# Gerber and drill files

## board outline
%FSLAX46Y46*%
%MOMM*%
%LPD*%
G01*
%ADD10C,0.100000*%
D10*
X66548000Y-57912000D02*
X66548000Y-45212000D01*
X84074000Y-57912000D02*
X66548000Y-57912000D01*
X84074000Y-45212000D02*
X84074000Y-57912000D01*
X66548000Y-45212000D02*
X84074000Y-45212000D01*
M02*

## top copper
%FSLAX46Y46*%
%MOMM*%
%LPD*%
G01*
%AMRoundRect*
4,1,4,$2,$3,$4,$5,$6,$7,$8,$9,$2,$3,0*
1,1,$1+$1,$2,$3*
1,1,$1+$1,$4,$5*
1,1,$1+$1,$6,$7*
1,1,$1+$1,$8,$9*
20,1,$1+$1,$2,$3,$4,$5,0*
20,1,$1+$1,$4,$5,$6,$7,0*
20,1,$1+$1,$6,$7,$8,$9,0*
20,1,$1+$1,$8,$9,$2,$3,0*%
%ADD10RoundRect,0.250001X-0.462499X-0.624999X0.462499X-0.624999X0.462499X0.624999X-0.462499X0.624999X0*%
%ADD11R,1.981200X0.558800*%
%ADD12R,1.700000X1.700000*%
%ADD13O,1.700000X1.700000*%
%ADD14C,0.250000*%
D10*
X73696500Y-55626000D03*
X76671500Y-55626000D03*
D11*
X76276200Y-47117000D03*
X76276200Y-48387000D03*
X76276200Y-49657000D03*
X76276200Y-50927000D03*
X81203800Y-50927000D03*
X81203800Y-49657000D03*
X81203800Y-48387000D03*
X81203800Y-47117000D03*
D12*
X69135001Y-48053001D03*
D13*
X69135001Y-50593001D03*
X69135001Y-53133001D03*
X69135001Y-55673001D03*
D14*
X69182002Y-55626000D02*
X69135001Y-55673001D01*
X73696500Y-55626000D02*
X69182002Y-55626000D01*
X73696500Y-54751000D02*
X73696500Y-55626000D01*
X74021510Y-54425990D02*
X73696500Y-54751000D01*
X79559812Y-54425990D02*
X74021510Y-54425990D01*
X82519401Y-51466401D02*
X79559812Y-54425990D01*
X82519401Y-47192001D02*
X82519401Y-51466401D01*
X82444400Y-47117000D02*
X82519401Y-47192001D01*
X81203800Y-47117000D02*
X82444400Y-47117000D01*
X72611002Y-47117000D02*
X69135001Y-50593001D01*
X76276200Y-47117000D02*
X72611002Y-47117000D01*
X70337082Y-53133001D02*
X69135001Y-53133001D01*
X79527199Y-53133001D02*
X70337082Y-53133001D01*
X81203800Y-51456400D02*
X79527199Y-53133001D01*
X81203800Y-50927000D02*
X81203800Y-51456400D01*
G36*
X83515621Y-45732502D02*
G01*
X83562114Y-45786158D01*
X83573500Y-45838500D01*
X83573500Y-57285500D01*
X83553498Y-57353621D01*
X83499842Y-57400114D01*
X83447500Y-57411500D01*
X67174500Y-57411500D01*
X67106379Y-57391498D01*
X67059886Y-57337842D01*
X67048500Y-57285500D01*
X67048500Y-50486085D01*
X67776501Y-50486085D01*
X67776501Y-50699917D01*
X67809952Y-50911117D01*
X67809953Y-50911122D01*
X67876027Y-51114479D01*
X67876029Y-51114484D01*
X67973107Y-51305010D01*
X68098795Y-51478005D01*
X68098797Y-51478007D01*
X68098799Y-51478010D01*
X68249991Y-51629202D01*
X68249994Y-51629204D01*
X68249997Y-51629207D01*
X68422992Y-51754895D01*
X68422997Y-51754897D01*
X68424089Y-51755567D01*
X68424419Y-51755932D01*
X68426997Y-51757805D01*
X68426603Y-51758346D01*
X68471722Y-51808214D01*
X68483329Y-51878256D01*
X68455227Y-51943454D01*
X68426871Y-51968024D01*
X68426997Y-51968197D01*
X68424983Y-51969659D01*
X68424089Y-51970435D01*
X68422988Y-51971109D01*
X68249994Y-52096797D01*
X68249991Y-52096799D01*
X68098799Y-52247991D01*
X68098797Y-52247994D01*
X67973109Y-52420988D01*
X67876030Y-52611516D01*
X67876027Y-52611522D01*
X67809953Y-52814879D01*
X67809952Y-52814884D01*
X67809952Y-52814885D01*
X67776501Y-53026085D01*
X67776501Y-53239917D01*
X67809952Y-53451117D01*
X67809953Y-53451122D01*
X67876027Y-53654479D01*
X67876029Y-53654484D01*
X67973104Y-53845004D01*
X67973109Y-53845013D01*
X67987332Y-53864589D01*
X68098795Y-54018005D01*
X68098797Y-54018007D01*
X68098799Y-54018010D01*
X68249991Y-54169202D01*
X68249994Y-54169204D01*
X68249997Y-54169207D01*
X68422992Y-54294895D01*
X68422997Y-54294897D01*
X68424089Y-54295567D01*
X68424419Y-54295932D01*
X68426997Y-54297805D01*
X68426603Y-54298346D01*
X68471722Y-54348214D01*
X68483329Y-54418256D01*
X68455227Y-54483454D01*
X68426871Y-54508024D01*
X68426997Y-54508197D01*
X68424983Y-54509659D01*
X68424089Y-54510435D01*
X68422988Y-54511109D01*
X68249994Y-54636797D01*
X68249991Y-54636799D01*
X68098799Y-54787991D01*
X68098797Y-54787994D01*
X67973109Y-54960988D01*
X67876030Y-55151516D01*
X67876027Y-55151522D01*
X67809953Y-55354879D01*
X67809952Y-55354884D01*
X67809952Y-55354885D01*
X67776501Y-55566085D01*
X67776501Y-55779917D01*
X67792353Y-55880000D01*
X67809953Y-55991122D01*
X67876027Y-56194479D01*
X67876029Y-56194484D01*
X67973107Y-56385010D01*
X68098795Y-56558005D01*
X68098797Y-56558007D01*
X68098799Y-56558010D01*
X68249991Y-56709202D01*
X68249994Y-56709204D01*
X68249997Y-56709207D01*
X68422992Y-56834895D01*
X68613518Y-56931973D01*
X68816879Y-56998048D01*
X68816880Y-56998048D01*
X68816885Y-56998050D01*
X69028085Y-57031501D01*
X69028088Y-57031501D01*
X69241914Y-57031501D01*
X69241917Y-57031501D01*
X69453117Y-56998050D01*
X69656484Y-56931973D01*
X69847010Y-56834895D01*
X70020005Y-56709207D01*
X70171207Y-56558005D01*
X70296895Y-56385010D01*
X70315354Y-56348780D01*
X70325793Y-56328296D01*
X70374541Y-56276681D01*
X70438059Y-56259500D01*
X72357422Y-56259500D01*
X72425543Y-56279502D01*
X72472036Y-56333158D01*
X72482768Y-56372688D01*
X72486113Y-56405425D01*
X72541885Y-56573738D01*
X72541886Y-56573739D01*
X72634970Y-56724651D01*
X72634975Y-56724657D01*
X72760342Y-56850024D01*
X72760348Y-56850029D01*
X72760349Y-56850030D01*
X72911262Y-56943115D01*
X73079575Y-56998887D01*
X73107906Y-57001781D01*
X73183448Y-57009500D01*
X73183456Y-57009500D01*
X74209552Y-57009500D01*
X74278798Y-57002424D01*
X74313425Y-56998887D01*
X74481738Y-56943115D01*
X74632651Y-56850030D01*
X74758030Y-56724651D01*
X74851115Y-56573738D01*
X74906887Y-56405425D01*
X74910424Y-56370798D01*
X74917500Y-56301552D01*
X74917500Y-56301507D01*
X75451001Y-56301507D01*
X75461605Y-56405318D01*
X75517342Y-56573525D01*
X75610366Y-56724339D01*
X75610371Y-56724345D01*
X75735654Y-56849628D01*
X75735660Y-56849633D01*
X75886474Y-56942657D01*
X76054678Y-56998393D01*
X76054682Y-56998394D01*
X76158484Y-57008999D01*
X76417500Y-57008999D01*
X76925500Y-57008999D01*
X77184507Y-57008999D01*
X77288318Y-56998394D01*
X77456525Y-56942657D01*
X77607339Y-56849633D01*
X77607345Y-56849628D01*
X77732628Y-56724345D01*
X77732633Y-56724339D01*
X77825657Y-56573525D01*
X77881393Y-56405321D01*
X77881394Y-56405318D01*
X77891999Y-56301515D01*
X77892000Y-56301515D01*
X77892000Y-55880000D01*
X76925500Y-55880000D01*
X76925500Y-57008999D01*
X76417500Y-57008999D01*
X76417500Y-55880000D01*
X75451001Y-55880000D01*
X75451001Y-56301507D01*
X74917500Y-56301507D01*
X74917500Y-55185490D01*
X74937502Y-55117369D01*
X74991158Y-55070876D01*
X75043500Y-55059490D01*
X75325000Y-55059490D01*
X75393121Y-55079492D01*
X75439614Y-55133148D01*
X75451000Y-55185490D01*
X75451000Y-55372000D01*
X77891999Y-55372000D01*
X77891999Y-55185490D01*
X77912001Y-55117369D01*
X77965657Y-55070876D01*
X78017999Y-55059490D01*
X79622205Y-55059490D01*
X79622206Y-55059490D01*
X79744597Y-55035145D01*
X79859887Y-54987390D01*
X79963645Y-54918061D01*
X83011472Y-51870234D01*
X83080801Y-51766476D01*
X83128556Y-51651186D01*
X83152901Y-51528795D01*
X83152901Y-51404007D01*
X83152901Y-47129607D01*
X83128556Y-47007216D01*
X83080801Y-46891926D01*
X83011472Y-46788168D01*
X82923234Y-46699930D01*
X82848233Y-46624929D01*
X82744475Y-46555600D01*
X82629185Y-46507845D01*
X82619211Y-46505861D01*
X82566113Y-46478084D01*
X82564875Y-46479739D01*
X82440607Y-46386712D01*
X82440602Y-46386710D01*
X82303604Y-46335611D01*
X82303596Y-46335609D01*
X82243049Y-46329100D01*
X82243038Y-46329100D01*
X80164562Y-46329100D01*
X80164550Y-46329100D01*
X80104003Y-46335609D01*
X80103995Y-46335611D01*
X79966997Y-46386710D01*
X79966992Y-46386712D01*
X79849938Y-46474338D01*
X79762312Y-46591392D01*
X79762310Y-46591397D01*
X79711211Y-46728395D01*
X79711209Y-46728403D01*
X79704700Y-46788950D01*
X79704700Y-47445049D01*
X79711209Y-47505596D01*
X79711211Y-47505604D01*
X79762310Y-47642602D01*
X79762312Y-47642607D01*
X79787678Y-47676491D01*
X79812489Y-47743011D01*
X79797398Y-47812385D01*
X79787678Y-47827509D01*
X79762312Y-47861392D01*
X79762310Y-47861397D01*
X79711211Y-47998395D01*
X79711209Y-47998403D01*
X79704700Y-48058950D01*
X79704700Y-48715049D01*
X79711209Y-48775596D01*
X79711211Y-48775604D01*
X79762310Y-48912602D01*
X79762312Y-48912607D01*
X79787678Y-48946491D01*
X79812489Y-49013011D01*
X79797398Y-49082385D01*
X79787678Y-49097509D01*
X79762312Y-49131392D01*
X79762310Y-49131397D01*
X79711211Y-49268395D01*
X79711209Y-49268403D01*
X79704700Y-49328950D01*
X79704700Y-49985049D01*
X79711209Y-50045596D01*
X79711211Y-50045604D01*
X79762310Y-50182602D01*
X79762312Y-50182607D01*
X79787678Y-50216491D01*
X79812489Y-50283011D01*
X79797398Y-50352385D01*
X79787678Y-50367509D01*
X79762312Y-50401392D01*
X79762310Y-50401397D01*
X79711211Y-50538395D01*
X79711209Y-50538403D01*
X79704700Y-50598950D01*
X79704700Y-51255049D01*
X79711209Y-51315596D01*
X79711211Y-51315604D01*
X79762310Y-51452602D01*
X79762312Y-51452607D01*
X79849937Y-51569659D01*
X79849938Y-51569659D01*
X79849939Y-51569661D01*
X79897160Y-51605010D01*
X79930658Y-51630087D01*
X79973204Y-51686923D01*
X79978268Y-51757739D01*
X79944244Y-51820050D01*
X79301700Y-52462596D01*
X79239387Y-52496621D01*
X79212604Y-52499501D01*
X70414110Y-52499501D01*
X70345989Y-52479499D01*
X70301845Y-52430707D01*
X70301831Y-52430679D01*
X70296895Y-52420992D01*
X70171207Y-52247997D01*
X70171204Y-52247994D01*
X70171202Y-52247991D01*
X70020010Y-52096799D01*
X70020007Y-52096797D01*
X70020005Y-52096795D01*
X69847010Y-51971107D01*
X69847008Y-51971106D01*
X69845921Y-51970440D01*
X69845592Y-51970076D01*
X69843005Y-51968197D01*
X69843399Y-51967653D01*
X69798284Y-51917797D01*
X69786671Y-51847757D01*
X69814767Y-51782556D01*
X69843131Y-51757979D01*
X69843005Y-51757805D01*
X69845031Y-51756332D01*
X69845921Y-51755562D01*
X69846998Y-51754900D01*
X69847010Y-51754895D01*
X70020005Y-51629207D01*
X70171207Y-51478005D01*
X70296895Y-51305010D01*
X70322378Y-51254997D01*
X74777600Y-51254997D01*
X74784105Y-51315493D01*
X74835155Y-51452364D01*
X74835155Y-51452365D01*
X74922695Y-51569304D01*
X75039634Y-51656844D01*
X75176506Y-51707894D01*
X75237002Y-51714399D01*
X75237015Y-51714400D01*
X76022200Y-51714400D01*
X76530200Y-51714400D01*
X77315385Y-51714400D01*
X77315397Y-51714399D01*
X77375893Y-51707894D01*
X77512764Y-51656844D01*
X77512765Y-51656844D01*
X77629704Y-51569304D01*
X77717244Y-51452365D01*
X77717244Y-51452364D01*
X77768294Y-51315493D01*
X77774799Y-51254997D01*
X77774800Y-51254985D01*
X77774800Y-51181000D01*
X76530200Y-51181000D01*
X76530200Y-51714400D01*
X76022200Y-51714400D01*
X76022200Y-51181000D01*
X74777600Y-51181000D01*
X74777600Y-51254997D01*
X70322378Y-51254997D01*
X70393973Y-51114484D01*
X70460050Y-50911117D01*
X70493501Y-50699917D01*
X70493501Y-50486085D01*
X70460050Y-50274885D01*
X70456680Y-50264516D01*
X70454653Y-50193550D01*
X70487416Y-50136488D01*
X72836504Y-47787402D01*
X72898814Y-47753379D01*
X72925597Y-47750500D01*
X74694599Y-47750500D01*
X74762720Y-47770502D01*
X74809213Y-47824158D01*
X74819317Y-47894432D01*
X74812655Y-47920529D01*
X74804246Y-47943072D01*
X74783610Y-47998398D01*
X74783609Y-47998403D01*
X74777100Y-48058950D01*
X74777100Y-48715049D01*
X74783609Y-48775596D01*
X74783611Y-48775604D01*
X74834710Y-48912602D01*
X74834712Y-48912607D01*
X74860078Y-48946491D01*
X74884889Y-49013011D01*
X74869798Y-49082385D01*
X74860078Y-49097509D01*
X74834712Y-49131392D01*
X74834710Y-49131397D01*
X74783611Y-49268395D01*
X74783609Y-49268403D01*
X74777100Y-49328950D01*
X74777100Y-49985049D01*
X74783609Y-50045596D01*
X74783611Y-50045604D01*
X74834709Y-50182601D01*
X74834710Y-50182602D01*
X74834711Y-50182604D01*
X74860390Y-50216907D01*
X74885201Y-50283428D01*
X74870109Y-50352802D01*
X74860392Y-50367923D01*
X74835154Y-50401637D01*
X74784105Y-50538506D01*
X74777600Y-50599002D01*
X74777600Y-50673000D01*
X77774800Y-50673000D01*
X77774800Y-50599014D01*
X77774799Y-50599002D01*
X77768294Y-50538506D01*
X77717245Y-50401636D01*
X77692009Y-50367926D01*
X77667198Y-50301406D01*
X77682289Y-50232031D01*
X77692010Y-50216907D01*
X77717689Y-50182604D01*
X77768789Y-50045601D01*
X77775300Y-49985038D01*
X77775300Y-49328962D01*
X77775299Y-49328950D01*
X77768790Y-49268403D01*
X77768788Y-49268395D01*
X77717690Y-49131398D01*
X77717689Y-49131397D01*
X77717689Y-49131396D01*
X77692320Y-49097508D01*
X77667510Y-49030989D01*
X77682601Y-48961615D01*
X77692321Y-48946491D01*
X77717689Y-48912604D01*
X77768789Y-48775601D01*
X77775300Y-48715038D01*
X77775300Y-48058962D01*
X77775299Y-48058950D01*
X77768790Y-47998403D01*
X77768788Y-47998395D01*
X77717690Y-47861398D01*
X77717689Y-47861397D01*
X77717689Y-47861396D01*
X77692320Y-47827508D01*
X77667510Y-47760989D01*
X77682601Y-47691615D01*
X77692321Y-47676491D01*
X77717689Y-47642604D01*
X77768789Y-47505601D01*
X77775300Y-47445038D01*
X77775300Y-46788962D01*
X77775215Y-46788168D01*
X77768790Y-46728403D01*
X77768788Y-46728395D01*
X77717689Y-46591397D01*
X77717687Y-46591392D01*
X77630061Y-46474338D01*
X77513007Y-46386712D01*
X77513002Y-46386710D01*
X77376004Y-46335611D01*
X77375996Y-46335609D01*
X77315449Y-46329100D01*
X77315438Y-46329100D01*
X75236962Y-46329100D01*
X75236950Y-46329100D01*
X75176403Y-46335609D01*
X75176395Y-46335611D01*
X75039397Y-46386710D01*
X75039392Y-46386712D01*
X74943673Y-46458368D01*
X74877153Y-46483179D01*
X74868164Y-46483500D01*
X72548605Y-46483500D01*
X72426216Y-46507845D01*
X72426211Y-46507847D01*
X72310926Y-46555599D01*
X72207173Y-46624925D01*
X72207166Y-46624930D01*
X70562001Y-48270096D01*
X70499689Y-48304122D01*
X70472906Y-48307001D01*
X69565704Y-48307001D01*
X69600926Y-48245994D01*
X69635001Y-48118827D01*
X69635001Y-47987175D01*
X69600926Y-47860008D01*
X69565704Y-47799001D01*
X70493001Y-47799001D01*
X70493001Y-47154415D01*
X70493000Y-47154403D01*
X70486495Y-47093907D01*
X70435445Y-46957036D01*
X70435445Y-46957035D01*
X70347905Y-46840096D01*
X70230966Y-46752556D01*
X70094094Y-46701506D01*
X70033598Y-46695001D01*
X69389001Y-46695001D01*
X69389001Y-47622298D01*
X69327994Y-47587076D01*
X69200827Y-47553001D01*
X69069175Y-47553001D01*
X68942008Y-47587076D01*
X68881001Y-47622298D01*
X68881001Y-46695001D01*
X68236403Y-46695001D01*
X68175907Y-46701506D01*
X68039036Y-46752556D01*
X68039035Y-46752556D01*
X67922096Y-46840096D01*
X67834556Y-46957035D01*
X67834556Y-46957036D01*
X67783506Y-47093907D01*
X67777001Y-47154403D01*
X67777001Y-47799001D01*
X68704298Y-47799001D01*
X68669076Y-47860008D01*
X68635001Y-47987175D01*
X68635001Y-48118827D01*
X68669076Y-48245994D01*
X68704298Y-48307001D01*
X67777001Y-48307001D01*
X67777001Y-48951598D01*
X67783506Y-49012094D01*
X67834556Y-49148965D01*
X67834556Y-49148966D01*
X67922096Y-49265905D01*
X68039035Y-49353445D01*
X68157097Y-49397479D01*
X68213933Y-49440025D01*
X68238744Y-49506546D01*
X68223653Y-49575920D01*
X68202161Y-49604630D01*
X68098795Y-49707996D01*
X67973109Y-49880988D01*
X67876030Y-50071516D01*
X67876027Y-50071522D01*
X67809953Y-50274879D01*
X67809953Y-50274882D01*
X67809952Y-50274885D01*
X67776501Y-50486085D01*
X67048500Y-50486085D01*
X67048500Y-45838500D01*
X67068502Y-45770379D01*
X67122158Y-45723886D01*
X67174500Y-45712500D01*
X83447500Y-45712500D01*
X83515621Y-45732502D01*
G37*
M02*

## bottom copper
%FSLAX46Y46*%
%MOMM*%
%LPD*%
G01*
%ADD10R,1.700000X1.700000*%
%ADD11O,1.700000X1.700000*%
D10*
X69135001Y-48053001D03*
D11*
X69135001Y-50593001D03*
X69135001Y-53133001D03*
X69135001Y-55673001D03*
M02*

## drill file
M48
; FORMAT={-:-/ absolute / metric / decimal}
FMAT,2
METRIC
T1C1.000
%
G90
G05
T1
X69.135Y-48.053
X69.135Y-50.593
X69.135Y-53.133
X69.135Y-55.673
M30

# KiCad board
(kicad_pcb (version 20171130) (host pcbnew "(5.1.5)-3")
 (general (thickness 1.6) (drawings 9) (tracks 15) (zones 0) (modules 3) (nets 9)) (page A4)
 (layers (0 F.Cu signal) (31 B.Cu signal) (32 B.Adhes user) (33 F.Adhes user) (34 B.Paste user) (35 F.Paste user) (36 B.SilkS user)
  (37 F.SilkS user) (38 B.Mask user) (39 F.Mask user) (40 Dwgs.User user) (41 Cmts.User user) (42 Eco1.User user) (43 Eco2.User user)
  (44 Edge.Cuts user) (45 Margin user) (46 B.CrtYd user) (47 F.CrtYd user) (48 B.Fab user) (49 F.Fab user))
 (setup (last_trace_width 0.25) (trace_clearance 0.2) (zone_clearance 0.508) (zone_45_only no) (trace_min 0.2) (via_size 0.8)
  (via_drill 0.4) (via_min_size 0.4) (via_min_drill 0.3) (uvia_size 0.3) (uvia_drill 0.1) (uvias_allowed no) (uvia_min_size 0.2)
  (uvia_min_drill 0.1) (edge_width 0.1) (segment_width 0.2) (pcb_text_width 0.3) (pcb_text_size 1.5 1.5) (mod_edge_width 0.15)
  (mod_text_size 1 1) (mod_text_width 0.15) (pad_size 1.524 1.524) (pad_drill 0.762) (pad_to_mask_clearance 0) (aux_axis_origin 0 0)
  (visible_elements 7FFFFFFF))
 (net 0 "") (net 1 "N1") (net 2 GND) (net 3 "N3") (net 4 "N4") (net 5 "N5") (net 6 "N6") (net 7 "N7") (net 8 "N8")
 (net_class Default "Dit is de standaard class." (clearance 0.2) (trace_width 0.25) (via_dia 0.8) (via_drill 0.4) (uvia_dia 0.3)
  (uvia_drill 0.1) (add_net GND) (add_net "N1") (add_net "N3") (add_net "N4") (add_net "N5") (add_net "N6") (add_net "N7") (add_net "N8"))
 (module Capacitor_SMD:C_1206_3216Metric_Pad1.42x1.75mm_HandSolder (layer F.Cu) (at 75.184 55.626)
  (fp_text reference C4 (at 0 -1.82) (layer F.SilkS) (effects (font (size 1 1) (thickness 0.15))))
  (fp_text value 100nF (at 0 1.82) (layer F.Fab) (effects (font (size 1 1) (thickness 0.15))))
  (pad 1 smd roundrect (at -1.4875 0) (size 1.425 1.75) (layers F.Cu F.Paste F.Mask) (roundrect_rratio 0.175439) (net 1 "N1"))
  (pad 2 smd roundrect (at 1.4875 0) (size 1.425 1.75) (layers F.Cu F.Paste F.Mask) (roundrect_rratio 0.175439) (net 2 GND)))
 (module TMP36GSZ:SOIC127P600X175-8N (layer F.Cu) (at 78.74 49.022)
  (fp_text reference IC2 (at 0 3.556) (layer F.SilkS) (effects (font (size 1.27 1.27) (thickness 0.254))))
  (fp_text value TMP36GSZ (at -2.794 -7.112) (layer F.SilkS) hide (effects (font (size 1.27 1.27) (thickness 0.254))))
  (pad 1 smd rect (at -2.4638 -1.905 90) (size 0.5588 1.9812) (layers F.Cu F.Paste F.Mask) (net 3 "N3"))
  (pad 2 smd rect (at -2.4638 -0.635 90) (size 0.5588 1.9812) (layers F.Cu F.Paste F.Mask) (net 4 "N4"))
  (pad 3 smd rect (at -2.4638 0.635 90) (size 0.5588 1.9812) (layers F.Cu F.Paste F.Mask) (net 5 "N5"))
  (pad 4 smd rect (at -2.4638 1.905 90) (size 0.5588 1.9812) (layers F.Cu F.Paste F.Mask) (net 2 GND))
  (pad 5 smd rect (at 2.4638 1.905 90) (size 0.5588 1.9812) (layers F.Cu F.Paste F.Mask) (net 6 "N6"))
  (pad 6 smd rect (at 2.4638 0.635 90) (size 0.5588 1.9812) (layers F.Cu F.Paste F.Mask) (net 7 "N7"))
  (pad 7 smd rect (at 2.4638 -0.635 90) (size 0.5588 1.9812) (layers F.Cu F.Paste F.Mask) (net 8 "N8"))
  (pad 8 smd rect (at 2.4638 -1.905 90) (size 0.5588 1.9812) (layers F.Cu F.Paste F.Mask) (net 1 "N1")))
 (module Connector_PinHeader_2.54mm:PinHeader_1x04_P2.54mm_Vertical (layer F.Cu) (at 69.135001 48.053001)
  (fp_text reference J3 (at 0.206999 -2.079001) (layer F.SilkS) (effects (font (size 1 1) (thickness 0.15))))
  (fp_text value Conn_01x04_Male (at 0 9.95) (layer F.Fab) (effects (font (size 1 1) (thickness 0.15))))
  (pad 1 thru_hole rect (at 0 0) (size 1.7 1.7) (drill 1) (layers *.Cu *.Mask) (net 2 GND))
  (pad 2 thru_hole oval (at 0 2.54) (size 1.7 1.7) (drill 1) (layers *.Cu *.Mask) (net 3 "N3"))
  (pad 3 thru_hole oval (at 0 5.08) (size 1.7 1.7) (drill 1) (layers *.Cu *.Mask) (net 6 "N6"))
  (pad 4 thru_hole oval (at 0 7.62) (size 1.7 1.7) (drill 1) (layers *.Cu *.Mask) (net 1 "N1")))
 (gr_line (start 66.548 57.912) (end 66.548 45.212) (layer Edge.Cuts) (width 0.1))
 (gr_line (start 84.074 57.912) (end 66.548 57.912) (layer Edge.Cuts) (width 0.1))
 (gr_line (start 84.074 45.212) (end 84.074 57.912) (layer Edge.Cuts) (width 0.1))
 (gr_line (start 66.548 45.212) (end 84.074 45.212) (layer Edge.Cuts) (width 0.1))
 (segment (start 69.182002 55.626) (end 69.135001 55.673001) (width 0.25) (layer F.Cu) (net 1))
 (segment (start 73.6965 55.626) (end 69.182002 55.626) (width 0.25) (layer F.Cu) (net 1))
 (segment (start 73.6965 54.751) (end 73.6965 55.626) (width 0.25) (layer F.Cu) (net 1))
 (segment (start 74.02151 54.42599) (end 73.6965 54.751) (width 0.25) (layer F.Cu) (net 1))
 (segment (start 79.559812 54.42599) (end 74.02151 54.42599) (width 0.25) (layer F.Cu) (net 1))
 (segment (start 82.519401 51.466401) (end 79.559812 54.42599) (width 0.25) (layer F.Cu) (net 1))
 (segment (start 82.519401 47.192001) (end 82.519401 51.466401) (width 0.25) (layer F.Cu) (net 1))
 (segment (start 82.4444 47.117) (end 82.519401 47.192001) (width 0.25) (layer F.Cu) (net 1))
 (segment (start 81.2038 47.117) (end 82.4444 47.117) (width 0.25) (layer F.Cu) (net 1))
 (segment (start 72.611002 47.117) (end 69.135001 50.593001) (width 0.25) (layer F.Cu) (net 3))
 (segment (start 76.2762 47.117) (end 72.611002 47.117) (width 0.25) (layer F.Cu) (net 3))
 (segment (start 70.337082 53.133001) (end 69.135001 53.133001) (width 0.25) (layer F.Cu) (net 6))
 (segment (start 79.527199 53.133001) (end 70.337082 53.133001) (width 0.25) (layer F.Cu) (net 6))
 (segment (start 81.2038 51.4564) (end 79.527199 53.133001) (width 0.25) (layer F.Cu) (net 6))
 (segment (start 81.2038 50.927) (end 81.2038 51.4564) (width 0.25) (layer F.Cu) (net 6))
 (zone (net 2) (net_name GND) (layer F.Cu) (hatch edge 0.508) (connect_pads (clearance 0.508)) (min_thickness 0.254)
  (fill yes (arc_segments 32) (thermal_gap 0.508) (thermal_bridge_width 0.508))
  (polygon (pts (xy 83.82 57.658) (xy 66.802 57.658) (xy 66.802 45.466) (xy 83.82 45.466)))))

